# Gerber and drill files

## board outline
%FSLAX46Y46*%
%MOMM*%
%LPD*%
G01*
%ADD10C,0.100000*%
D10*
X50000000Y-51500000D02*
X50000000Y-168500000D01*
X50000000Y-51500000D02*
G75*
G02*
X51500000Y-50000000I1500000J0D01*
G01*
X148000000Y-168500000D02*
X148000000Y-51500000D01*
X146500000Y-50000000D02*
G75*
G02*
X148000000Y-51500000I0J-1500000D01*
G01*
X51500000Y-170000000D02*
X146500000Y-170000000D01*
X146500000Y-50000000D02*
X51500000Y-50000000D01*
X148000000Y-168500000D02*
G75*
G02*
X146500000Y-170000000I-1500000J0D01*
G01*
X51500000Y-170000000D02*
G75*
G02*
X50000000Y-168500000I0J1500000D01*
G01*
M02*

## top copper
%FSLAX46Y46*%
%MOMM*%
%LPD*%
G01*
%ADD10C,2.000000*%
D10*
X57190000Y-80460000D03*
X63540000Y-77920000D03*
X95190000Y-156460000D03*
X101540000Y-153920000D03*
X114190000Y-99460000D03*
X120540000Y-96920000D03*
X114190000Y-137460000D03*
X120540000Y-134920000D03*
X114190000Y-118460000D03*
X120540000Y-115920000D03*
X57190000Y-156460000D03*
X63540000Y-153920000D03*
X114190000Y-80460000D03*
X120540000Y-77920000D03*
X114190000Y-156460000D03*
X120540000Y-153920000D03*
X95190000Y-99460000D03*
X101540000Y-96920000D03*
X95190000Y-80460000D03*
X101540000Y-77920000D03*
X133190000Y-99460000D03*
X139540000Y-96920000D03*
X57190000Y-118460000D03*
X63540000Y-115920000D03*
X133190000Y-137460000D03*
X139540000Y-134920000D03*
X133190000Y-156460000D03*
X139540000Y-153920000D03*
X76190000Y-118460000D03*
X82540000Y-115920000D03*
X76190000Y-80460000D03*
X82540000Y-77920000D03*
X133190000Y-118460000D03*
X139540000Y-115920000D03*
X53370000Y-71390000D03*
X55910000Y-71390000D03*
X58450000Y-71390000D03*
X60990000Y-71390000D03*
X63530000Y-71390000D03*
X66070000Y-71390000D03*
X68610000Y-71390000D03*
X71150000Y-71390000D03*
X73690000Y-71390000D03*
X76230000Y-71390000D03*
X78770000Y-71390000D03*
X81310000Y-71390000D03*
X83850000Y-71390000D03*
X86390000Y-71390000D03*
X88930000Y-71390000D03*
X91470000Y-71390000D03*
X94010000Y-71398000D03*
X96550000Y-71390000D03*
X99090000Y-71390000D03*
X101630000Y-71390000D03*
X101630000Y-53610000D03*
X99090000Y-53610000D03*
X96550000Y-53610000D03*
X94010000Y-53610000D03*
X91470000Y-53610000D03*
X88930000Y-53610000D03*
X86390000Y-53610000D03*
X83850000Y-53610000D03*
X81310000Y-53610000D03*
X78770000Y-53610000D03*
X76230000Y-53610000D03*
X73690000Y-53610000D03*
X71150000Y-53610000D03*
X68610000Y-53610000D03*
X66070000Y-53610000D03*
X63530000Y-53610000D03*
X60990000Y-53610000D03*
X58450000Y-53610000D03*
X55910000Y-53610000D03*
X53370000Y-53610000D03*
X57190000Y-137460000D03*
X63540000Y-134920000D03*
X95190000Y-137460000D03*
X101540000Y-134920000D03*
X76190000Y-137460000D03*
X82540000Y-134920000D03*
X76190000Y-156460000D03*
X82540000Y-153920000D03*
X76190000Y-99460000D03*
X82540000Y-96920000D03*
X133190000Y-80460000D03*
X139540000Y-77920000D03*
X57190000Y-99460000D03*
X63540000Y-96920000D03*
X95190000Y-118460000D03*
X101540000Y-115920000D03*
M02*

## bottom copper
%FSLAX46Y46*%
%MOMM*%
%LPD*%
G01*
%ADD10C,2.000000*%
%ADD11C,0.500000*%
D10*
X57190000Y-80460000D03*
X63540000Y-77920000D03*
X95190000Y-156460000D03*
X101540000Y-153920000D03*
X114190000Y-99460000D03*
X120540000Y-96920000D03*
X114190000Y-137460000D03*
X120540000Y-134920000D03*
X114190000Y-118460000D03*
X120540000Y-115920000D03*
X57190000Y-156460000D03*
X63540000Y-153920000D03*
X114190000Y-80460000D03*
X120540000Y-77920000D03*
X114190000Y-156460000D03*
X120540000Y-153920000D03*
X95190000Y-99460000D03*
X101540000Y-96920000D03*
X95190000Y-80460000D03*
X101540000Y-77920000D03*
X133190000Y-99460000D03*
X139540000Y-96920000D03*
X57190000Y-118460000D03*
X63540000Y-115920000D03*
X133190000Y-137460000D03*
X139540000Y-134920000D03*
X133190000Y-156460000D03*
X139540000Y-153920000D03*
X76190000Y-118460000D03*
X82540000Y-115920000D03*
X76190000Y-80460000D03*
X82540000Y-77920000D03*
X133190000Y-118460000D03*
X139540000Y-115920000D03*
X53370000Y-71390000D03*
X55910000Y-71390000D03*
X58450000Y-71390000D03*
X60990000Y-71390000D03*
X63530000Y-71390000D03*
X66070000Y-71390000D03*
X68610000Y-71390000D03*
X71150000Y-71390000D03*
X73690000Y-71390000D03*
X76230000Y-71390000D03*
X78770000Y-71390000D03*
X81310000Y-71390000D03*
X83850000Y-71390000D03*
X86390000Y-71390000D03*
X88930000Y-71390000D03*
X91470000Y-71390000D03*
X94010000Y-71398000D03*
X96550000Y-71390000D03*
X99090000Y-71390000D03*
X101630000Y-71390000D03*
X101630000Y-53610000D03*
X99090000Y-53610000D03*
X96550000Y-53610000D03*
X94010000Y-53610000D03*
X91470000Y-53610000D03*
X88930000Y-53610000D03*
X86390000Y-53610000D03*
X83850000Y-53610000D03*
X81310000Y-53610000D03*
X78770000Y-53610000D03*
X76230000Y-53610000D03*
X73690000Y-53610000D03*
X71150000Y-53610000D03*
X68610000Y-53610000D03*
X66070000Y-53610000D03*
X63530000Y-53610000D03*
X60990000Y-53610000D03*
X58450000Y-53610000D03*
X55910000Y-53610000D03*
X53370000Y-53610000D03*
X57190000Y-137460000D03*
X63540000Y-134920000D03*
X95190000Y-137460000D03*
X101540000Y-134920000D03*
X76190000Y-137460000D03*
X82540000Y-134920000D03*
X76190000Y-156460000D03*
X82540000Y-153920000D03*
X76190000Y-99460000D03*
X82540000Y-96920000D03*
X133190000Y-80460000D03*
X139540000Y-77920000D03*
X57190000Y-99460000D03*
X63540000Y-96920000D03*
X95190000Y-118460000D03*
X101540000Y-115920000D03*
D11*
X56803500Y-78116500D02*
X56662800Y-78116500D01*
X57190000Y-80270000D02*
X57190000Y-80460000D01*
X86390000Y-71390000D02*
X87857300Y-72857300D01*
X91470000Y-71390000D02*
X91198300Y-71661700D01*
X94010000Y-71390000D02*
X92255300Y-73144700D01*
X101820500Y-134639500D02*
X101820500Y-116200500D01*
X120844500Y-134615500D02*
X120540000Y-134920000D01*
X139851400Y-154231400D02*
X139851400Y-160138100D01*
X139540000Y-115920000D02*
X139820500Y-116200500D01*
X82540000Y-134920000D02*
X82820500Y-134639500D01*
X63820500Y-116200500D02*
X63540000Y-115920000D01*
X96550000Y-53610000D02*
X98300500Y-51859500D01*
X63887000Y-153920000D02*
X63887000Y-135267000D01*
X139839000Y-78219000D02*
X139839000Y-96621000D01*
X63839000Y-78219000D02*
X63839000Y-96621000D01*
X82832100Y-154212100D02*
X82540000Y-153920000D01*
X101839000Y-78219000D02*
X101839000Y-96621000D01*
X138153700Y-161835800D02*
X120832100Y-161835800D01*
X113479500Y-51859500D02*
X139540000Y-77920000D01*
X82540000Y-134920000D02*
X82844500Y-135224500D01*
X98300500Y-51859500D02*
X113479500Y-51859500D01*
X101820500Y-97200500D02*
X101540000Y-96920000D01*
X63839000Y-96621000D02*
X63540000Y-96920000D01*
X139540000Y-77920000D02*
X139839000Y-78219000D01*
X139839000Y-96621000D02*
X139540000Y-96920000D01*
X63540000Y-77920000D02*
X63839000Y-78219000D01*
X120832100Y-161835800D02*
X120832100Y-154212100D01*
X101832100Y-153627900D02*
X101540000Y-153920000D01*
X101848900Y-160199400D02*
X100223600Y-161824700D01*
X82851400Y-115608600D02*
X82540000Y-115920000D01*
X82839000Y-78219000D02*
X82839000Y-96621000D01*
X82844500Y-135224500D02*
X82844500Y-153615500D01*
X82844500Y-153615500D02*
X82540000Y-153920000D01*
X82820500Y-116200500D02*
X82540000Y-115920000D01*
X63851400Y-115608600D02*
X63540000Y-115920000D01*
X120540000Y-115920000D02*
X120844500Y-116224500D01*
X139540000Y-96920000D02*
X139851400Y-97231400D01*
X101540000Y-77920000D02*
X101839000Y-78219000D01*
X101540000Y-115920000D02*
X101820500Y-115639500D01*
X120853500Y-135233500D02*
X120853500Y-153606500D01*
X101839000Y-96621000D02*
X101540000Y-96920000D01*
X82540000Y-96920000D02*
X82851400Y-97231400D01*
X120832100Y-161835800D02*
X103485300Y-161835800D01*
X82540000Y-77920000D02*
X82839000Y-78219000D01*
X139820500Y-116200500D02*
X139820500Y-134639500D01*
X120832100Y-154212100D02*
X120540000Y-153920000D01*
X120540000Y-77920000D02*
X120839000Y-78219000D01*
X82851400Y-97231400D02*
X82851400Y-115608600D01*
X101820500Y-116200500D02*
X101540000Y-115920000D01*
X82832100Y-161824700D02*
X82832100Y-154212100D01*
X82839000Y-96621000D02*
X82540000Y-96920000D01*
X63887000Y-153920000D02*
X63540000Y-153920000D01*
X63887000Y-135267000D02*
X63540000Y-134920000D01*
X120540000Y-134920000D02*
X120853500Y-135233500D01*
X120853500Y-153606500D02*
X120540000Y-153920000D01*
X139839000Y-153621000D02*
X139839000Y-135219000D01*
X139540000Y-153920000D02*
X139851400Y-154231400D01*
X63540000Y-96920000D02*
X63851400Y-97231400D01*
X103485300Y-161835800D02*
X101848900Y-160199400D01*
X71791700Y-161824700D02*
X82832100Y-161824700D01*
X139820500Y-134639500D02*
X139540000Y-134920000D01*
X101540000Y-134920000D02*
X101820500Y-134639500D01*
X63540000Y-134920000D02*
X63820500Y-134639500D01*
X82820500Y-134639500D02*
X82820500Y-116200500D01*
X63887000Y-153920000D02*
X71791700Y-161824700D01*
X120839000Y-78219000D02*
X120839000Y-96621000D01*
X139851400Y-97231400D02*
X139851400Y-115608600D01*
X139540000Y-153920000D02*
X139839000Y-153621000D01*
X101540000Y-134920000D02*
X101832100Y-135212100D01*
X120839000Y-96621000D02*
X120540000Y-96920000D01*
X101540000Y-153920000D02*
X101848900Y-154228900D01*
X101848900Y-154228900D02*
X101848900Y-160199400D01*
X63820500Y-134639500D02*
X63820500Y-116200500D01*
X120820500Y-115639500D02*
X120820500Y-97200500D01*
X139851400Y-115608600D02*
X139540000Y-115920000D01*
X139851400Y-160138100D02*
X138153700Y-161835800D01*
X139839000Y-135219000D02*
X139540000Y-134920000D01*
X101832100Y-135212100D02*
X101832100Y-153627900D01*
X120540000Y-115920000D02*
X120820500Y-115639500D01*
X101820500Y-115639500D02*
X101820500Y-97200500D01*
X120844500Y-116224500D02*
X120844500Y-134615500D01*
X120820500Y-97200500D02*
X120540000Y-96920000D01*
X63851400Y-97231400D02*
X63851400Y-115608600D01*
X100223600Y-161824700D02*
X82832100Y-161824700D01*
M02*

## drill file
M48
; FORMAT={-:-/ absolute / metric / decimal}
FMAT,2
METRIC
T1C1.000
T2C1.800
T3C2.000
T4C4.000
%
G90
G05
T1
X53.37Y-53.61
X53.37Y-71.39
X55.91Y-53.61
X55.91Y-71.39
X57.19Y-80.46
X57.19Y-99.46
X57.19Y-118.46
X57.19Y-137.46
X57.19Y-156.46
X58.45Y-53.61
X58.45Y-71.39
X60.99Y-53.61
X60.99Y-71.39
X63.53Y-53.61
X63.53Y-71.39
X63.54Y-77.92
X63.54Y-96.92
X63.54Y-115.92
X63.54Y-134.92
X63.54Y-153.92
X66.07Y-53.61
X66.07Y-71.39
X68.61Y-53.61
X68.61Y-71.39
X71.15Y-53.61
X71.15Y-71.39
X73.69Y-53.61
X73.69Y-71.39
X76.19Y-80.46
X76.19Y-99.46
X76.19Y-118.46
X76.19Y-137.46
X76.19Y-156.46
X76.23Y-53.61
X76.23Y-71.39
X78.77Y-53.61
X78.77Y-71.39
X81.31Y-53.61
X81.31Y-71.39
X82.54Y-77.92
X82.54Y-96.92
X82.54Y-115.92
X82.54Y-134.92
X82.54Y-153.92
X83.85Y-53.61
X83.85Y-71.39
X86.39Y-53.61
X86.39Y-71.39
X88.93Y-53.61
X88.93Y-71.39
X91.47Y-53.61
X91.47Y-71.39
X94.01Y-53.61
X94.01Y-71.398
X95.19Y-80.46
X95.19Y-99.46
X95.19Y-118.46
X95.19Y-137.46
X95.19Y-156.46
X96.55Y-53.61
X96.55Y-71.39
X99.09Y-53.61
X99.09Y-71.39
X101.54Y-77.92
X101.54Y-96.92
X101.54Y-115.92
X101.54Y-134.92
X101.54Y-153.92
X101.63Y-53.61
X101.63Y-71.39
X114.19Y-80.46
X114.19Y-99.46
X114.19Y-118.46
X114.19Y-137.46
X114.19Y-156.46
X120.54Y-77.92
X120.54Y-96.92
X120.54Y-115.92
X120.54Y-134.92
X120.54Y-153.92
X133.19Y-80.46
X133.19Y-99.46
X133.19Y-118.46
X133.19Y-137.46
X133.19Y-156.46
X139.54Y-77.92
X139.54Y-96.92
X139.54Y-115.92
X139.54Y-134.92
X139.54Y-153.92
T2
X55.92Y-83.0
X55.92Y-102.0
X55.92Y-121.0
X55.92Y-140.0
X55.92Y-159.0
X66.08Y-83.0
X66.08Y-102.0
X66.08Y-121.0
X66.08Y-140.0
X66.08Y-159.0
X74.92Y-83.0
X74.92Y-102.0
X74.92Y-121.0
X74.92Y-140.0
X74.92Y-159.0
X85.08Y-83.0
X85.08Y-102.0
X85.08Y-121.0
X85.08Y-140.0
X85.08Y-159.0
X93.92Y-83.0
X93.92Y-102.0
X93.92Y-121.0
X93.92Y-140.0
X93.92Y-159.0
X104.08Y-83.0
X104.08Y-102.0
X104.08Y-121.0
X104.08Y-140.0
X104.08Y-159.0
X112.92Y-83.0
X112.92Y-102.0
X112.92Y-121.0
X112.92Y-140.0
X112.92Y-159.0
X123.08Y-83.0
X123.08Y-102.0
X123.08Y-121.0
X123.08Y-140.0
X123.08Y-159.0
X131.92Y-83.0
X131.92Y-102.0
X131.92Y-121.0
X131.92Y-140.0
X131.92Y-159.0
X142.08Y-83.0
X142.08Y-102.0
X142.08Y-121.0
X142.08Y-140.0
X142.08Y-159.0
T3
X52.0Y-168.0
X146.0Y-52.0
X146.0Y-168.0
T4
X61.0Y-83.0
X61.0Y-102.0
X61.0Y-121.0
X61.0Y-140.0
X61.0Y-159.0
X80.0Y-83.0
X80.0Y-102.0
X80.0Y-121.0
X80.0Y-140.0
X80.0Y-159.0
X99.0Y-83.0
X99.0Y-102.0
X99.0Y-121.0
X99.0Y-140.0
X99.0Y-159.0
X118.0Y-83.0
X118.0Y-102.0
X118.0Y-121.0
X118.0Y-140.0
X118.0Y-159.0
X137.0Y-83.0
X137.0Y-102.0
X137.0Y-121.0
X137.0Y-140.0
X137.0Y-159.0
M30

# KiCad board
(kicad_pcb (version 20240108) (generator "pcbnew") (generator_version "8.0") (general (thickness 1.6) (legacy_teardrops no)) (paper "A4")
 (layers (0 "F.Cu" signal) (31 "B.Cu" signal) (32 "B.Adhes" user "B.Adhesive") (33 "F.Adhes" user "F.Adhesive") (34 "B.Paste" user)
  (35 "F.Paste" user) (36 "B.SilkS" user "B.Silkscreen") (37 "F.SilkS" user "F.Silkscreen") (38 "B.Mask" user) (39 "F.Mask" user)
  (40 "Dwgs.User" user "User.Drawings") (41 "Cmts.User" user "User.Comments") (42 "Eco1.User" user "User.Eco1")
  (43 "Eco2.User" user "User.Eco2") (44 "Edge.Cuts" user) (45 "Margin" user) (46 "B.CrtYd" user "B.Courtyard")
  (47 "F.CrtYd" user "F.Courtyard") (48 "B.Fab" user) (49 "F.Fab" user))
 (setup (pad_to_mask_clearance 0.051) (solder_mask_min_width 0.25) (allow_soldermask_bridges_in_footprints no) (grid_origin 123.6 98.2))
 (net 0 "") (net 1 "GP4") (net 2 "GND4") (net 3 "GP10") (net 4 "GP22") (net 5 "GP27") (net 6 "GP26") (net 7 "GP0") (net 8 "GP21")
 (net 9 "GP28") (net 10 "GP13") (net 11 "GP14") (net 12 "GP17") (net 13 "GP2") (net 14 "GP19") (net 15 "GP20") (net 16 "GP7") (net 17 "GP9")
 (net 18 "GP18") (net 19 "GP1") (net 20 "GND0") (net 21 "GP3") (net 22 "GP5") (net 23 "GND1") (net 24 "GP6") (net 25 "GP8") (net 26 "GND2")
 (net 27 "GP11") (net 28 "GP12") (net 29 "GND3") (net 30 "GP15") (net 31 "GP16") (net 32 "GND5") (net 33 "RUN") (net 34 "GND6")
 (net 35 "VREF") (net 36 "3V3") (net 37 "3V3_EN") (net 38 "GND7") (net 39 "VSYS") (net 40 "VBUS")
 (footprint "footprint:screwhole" (layer "F.Cu") (at 146 52)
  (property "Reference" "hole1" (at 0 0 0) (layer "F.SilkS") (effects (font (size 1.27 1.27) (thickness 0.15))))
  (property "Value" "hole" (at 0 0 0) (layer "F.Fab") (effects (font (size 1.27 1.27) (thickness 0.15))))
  (pad "" np_thru_hole circle (at 0 0) (size 2 2) (drill 2) (layers "*.Cu" "*.Mask")))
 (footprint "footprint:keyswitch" (layer "F.Cu") (at 61 83)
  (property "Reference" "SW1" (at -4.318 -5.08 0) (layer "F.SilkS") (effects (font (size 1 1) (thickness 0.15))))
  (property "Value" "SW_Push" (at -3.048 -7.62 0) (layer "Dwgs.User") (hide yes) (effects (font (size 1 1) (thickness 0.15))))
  (pad "" np_thru_hole circle (at -5.08 0) (size 1.8 1.8) (drill 1.8) (layers "*.Cu" "*.Mask"))
  (pad "" np_thru_hole circle (at 0 0) (size 4 4) (drill 4) (layers "*.Cu" "*.Mask"))
  (pad "" np_thru_hole circle (at 5.08 0) (size 1.8 1.8) (drill 1.8) (layers "*.Cu" "*.Mask"))
  (pad "1" thru_hole circle (at -3.81 -2.54) (size 2 2) (drill 1) (layers "*.Cu" "*.Mask") (remove_unused_layers no) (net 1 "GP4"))
  (pad "2" thru_hole circle (at 2.54 -5.08) (size 2 2) (drill 1) (layers "*.Cu" "*.Mask") (remove_unused_layers no) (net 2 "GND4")))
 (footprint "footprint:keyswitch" (layer "F.Cu") (at 99 159)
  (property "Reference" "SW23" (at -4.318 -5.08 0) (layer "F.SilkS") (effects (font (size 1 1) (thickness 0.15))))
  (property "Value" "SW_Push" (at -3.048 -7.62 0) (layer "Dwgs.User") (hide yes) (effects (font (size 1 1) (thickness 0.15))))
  (pad "" np_thru_hole circle (at -5.08 0) (size 1.8 1.8) (drill 1.8) (layers "*.Cu" "*.Mask"))
  (pad "" np_thru_hole circle (at 0 0) (size 4 4) (drill 4) (layers "*.Cu" "*.Mask"))
  (pad "" np_thru_hole circle (at 5.08 0) (size 1.8 1.8) (drill 1.8) (layers "*.Cu" "*.Mask"))
  (pad "1" thru_hole circle (at -3.81 -2.54) (size 2 2) (drill 1) (layers "*.Cu" "*.Mask") (remove_unused_layers no) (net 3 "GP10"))
  (pad "2" thru_hole circle (at 2.54 -5.08) (size 2 2) (drill 1) (layers "*.Cu" "*.Mask") (remove_unused_layers no) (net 2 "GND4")))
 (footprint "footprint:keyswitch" (layer "F.Cu") (at 118 102)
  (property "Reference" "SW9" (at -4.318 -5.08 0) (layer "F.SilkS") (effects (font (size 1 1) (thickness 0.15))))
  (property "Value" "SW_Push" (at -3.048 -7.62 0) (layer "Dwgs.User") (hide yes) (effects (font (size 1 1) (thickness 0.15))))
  (pad "" np_thru_hole circle (at -5.08 0) (size 1.8 1.8) (drill 1.8) (layers "*.Cu" "*.Mask"))
  (pad "" np_thru_hole circle (at 0 0) (size 4 4) (drill 4) (layers "*.Cu" "*.Mask"))
  (pad "" np_thru_hole circle (at 5.08 0) (size 1.8 1.8) (drill 1.8) (layers "*.Cu" "*.Mask"))
  (pad "1" thru_hole circle (at -3.81 -2.54) (size 2 2) (drill 1) (layers "*.Cu" "*.Mask") (remove_unused_layers no) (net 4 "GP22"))
  (pad "2" thru_hole circle (at 2.54 -5.08) (size 2 2) (drill 1) (layers "*.Cu" "*.Mask") (remove_unused_layers no) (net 2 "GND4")))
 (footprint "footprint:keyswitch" (layer "F.Cu") (at 118 140)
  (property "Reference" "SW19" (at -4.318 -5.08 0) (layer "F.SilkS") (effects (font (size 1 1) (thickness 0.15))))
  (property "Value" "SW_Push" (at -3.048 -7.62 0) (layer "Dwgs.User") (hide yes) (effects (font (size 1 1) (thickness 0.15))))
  (pad "" np_thru_hole circle (at -5.08 0) (size 1.8 1.8) (drill 1.8) (layers "*.Cu" "*.Mask"))
  (pad "" np_thru_hole circle (at 0 0) (size 4 4) (drill 4) (layers "*.Cu" "*.Mask"))
  (pad "" np_thru_hole circle (at 5.08 0) (size 1.8 1.8) (drill 1.8) (layers "*.Cu" "*.Mask"))
  (pad "1" thru_hole circle (at -3.81 -2.54) (size 2 2) (drill 1) (layers "*.Cu" "*.Mask") (remove_unused_layers no) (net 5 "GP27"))
  (pad "2" thru_hole circle (at 2.54 -5.08) (size 2 2) (drill 1) (layers "*.Cu" "*.Mask") (remove_unused_layers no) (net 2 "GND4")))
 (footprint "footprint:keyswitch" (layer "F.Cu") (at 118 121)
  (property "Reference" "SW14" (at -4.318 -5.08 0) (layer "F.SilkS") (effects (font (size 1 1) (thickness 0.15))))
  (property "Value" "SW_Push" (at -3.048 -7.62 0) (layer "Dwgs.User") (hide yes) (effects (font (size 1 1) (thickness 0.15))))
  (pad "" np_thru_hole circle (at -5.08 0) (size 1.8 1.8) (drill 1.8) (layers "*.Cu" "*.Mask"))
  (pad "" np_thru_hole circle (at 0 0) (size 4 4) (drill 4) (layers "*.Cu" "*.Mask"))
  (pad "" np_thru_hole circle (at 5.08 0) (size 1.8 1.8) (drill 1.8) (layers "*.Cu" "*.Mask"))
  (pad "1" thru_hole circle (at -3.81 -2.54) (size 2 2) (drill 1) (layers "*.Cu" "*.Mask") (remove_unused_layers no) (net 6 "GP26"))
  (pad "2" thru_hole circle (at 2.54 -5.08) (size 2 2) (drill 1) (layers "*.Cu" "*.Mask") (remove_unused_layers no) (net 2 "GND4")))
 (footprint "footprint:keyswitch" (layer "F.Cu") (at 61 159)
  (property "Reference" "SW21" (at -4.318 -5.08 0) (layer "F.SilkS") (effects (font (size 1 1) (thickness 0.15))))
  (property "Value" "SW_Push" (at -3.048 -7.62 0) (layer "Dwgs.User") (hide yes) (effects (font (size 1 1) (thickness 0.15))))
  (pad "" np_thru_hole circle (at -5.08 0) (size 1.8 1.8) (drill 1.8) (layers "*.Cu" "*.Mask"))
  (pad "" np_thru_hole circle (at 0 0) (size 4 4) (drill 4) (layers "*.Cu" "*.Mask"))
  (pad "" np_thru_hole circle (at 5.08 0) (size 1.8 1.8) (drill 1.8) (layers "*.Cu" "*.Mask"))
  (pad "1" thru_hole circle (at -3.81 -2.54) (size 2 2) (drill 1) (layers "*.Cu" "*.Mask") (remove_unused_layers no) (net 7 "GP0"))
  (pad "2" thru_hole circle (at 2.54 -5.08) (size 2 2) (drill 1) (layers "*.Cu" "*.Mask") (remove_unused_layers no) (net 2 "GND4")))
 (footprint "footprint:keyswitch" (layer "F.Cu") (at 118 83)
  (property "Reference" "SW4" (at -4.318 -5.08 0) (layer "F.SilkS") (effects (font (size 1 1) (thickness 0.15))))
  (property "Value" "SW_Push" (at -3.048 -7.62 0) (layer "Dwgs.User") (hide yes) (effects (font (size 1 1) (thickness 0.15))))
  (pad "" np_thru_hole circle (at -5.08 0) (size 1.8 1.8) (drill 1.8) (layers "*.Cu" "*.Mask"))
  (pad "" np_thru_hole circle (at 0 0) (size 4 4) (drill 4) (layers "*.Cu" "*.Mask"))
  (pad "" np_thru_hole circle (at 5.08 0) (size 1.8 1.8) (drill 1.8) (layers "*.Cu" "*.Mask"))
  (pad "1" thru_hole circle (at -3.81 -2.54) (size 2 2) (drill 1) (layers "*.Cu" "*.Mask") (remove_unused_layers no) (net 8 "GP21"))
  (pad "2" thru_hole circle (at 2.54 -5.08) (size 2 2) (drill 1) (layers "*.Cu" "*.Mask") (remove_unused_layers no) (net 2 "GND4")))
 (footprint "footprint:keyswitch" (layer "F.Cu") (at 118 159)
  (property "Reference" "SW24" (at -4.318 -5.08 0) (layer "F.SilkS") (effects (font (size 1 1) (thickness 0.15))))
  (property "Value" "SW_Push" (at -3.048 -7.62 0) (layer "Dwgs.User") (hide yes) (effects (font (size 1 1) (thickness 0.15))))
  (pad "" np_thru_hole circle (at -5.08 0) (size 1.8 1.8) (drill 1.8) (layers "*.Cu" "*.Mask"))
  (pad "" np_thru_hole circle (at 0 0) (size 4 4) (drill 4) (layers "*.Cu" "*.Mask"))
  (pad "" np_thru_hole circle (at 5.08 0) (size 1.8 1.8) (drill 1.8) (layers "*.Cu" "*.Mask"))
  (pad "1" thru_hole circle (at -3.81 -2.54) (size 2 2) (drill 1) (layers "*.Cu" "*.Mask") (remove_unused_layers no) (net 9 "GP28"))
  (pad "2" thru_hole circle (at 2.54 -5.08) (size 2 2) (drill 1) (layers "*.Cu" "*.Mask") (remove_unused_layers no) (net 2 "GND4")))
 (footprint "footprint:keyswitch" (layer "F.Cu") (at 99 102)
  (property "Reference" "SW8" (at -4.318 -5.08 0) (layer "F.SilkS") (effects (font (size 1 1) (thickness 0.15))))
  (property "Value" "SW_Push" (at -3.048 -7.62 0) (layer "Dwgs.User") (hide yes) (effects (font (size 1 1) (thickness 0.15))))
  (pad "" np_thru_hole circle (at -5.08 0) (size 1.8 1.8) (drill 1.8) (layers "*.Cu" "*.Mask"))
  (pad "" np_thru_hole circle (at 0 0) (size 4 4) (drill 4) (layers "*.Cu" "*.Mask"))
  (pad "" np_thru_hole circle (at 5.08 0) (size 1.8 1.8) (drill 1.8) (layers "*.Cu" "*.Mask"))
  (pad "1" thru_hole circle (at -3.81 -2.54) (size 2 2) (drill 1) (layers "*.Cu" "*.Mask") (remove_unused_layers no) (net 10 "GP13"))
  (pad "2" thru_hole circle (at 2.54 -5.08) (size 2 2) (drill 1) (layers "*.Cu" "*.Mask") (remove_unused_layers no) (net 2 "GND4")))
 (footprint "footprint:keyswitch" (layer "F.Cu") (at 99 83)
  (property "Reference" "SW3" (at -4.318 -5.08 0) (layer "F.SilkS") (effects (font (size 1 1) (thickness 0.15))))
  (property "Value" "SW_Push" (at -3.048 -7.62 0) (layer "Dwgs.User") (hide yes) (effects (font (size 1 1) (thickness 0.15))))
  (pad "" np_thru_hole circle (at -5.08 0) (size 1.8 1.8) (drill 1.8) (layers "*.Cu" "*.Mask"))
  (pad "" np_thru_hole circle (at 0 0) (size 4 4) (drill 4) (layers "*.Cu" "*.Mask"))
  (pad "" np_thru_hole circle (at 5.08 0) (size 1.8 1.8) (drill 1.8) (layers "*.Cu" "*.Mask"))
  (pad "1" thru_hole circle (at -3.81 -2.54) (size 2 2) (drill 1) (layers "*.Cu" "*.Mask") (remove_unused_layers no) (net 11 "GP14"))
  (pad "2" thru_hole circle (at 2.54 -5.08) (size 2 2) (drill 1) (layers "*.Cu" "*.Mask") (remove_unused_layers no) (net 2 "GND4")))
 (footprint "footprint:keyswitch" (layer "F.Cu") (at 137 102)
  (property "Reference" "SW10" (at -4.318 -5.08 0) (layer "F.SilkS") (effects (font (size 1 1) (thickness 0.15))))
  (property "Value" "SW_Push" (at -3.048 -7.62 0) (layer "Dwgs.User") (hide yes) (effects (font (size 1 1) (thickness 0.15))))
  (pad "" np_thru_hole circle (at -5.08 0) (size 1.8 1.8) (drill 1.8) (layers "*.Cu" "*.Mask"))
  (pad "" np_thru_hole circle (at 0 0) (size 4 4) (drill 4) (layers "*.Cu" "*.Mask"))
  (pad "" np_thru_hole circle (at 5.08 0) (size 1.8 1.8) (drill 1.8) (layers "*.Cu" "*.Mask"))
  (pad "1" thru_hole circle (at -3.81 -2.54) (size 2 2) (drill 1) (layers "*.Cu" "*.Mask") (remove_unused_layers no) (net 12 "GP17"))
  (pad "2" thru_hole circle (at 2.54 -5.08) (size 2 2) (drill 1) (layers "*.Cu" "*.Mask") (remove_unused_layers no) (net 2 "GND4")))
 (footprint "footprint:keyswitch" (layer "F.Cu") (at 61 121)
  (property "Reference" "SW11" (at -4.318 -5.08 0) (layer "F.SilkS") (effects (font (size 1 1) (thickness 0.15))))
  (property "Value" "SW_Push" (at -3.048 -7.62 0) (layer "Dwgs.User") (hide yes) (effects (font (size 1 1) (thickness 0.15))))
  (pad "" np_thru_hole circle (at -5.08 0) (size 1.8 1.8) (drill 1.8) (layers "*.Cu" "*.Mask"))
  (pad "" np_thru_hole circle (at 0 0) (size 4 4) (drill 4) (layers "*.Cu" "*.Mask"))
  (pad "" np_thru_hole circle (at 5.08 0) (size 1.8 1.8) (drill 1.8) (layers "*.Cu" "*.Mask"))
  (pad "1" thru_hole circle (at -3.81 -2.54) (size 2 2) (drill 1) (layers "*.Cu" "*.Mask") (remove_unused_layers no) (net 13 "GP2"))
  (pad "2" thru_hole circle (at 2.54 -5.08) (size 2 2) (drill 1) (layers "*.Cu" "*.Mask") (remove_unused_layers no) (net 2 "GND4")))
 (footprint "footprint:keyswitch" (layer "F.Cu") (at 137 140)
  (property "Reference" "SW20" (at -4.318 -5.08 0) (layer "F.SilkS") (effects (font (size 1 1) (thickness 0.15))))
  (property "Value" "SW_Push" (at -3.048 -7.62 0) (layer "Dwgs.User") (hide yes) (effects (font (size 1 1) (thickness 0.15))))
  (pad "" np_thru_hole circle (at -5.08 0) (size 1.8 1.8) (drill 1.8) (layers "*.Cu" "*.Mask"))
  (pad "" np_thru_hole circle (at 0 0) (size 4 4) (drill 4) (layers "*.Cu" "*.Mask"))
  (pad "" np_thru_hole circle (at 5.08 0) (size 1.8 1.8) (drill 1.8) (layers "*.Cu" "*.Mask"))
  (pad "1" thru_hole circle (at -3.81 -2.54) (size 2 2) (drill 1) (layers "*.Cu" "*.Mask") (remove_unused_layers no) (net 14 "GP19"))
  (pad "2" thru_hole circle (at 2.54 -5.08) (size 2 2) (drill 1) (layers "*.Cu" "*.Mask") (remove_unused_layers no) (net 2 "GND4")))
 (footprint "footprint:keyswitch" (layer "F.Cu") (at 137 159)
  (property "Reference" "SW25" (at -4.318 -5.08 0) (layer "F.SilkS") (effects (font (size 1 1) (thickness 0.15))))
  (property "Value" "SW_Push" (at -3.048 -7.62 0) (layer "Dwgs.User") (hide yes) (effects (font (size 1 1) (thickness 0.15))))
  (pad "" np_thru_hole circle (at -5.08 0) (size 1.8 1.8) (drill 1.8) (layers "*.Cu" "*.Mask"))
  (pad "" np_thru_hole circle (at 0 0) (size 4 4) (drill 4) (layers "*.Cu" "*.Mask"))
  (pad "" np_thru_hole circle (at 5.08 0) (size 1.8 1.8) (drill 1.8) (layers "*.Cu" "*.Mask"))
  (pad "1" thru_hole circle (at -3.81 -2.54) (size 2 2) (drill 1) (layers "*.Cu" "*.Mask") (remove_unused_layers no) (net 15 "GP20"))
  (pad "2" thru_hole circle (at 2.54 -5.08) (size 2 2) (drill 1) (layers "*.Cu" "*.Mask") (remove_unused_layers no) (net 2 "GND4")))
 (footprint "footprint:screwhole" (layer "F.Cu") (at 52 168)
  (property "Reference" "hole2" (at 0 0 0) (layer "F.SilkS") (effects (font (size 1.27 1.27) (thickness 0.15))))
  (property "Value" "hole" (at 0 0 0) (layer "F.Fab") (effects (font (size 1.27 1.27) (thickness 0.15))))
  (pad "" np_thru_hole circle (at 0 0) (size 2 2) (drill 2) (layers "*.Cu" "*.Mask")))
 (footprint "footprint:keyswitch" (layer "F.Cu") (at 80 121)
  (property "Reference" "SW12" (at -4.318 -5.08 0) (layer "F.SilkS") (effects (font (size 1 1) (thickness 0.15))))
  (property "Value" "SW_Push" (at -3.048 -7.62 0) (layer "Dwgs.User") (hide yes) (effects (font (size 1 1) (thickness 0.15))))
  (pad "" np_thru_hole circle (at -5.08 0) (size 1.8 1.8) (drill 1.8) (layers "*.Cu" "*.Mask"))
  (pad "" np_thru_hole circle (at 0 0) (size 4 4) (drill 4) (layers "*.Cu" "*.Mask"))
  (pad "" np_thru_hole circle (at 5.08 0) (size 1.8 1.8) (drill 1.8) (layers "*.Cu" "*.Mask"))
  (pad "1" thru_hole circle (at -3.81 -2.54) (size 2 2) (drill 1) (layers "*.Cu" "*.Mask") (remove_unused_layers no) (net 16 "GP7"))
  (pad "2" thru_hole circle (at 2.54 -5.08) (size 2 2) (drill 1) (layers "*.Cu" "*.Mask") (remove_unused_layers no) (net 2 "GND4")))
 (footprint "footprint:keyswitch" (layer "F.Cu") (at 80 83)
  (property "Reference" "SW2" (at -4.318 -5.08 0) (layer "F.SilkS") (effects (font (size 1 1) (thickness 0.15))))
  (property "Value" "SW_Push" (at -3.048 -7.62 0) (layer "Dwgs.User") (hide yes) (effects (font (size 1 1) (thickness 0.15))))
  (pad "" np_thru_hole circle (at -5.08 0) (size 1.8 1.8) (drill 1.8) (layers "*.Cu" "*.Mask"))
  (pad "" np_thru_hole circle (at 0 0) (size 4 4) (drill 4) (layers "*.Cu" "*.Mask"))
  (pad "" np_thru_hole circle (at 5.08 0) (size 1.8 1.8) (drill 1.8) (layers "*.Cu" "*.Mask"))
  (pad "1" thru_hole circle (at -3.81 -2.54) (size 2 2) (drill 1) (layers "*.Cu" "*.Mask") (remove_unused_layers no) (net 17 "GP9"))
  (pad "2" thru_hole circle (at 2.54 -5.08) (size 2 2) (drill 1) (layers "*.Cu" "*.Mask") (remove_unused_layers no) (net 2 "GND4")))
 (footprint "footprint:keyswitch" (layer "F.Cu") (at 137 121)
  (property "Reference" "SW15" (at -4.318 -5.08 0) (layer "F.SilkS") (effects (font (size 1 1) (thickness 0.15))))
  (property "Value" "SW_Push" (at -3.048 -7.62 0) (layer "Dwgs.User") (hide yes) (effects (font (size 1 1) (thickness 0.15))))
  (pad "" np_thru_hole circle (at -5.08 0) (size 1.8 1.8) (drill 1.8) (layers "*.Cu" "*.Mask"))
  (pad "" np_thru_hole circle (at 0 0) (size 4 4) (drill 4) (layers "*.Cu" "*.Mask"))
  (pad "" np_thru_hole circle (at 5.08 0) (size 1.8 1.8) (drill 1.8) (layers "*.Cu" "*.Mask"))
  (pad "1" thru_hole circle (at -3.81 -2.54) (size 2 2) (drill 1) (layers "*.Cu" "*.Mask") (remove_unused_layers no) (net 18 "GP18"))
  (pad "2" thru_hole circle (at 2.54 -5.08) (size 2 2) (drill 1) (layers "*.Cu" "*.Mask") (remove_unused_layers no) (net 2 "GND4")))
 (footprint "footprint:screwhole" (layer "F.Cu") (at 146 168)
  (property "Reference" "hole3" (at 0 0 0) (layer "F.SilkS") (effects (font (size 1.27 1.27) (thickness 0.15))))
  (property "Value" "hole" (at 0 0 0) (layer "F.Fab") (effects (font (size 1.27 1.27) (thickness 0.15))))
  (pad "" np_thru_hole circle (at 0 0) (size 2 2) (drill 2) (layers "*.Cu" "*.Mask")))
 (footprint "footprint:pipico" (layer "F.Cu") (at 77.5 62.5)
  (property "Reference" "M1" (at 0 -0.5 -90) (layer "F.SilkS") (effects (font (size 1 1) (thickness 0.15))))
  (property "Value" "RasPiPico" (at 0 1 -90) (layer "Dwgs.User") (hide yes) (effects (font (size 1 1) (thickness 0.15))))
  (pad "1" thru_hole circle (at -24.13 8.89 270) (size 2 2) (drill 1) (layers "*.Cu" "*.Mask") (remove_unused_layers no) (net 7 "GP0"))
  (pad "2" thru_hole circle (at -21.59 8.89 270) (size 2 2) (drill 1) (layers "*.Cu" "*.Mask") (remove_unused_layers no) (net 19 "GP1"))
  (pad "3" thru_hole circle (at -19.05 8.89 270) (size 2 2) (drill 1) (layers "*.Cu" "*.Mask") (remove_unused_layers no) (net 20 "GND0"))
  (pad "4" thru_hole circle (at -16.51 8.89 270) (size 2 2) (drill 1) (layers "*.Cu" "*.Mask") (remove_unused_layers no) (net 13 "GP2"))
  (pad "5" thru_hole circle (at -13.97 8.89 270) (size 2 2) (drill 1) (layers "*.Cu" "*.Mask") (remove_unused_layers no) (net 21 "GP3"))
  (pad "6" thru_hole circle (at -11.43 8.89 270) (size 2 2) (drill 1) (layers "*.Cu" "*.Mask") (remove_unused_layers no) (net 1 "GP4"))
  (pad "7" thru_hole circle (at -8.89 8.89 270) (size 2 2) (drill 1) (layers "*.Cu" "*.Mask") (remove_unused_layers no) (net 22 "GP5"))
  (pad "8" thru_hole circle (at -6.35 8.89 270) (size 2 2) (drill 1) (layers "*.Cu" "*.Mask") (remove_unused_layers no) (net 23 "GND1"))
  (pad "9" thru_hole circle (at -3.81 8.89 270) (size 2 2) (drill 1) (layers "*.Cu" "*.Mask") (remove_unused_layers no) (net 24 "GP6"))
  (pad "10" thru_hole circle (at -1.27 8.89 270) (size 2 2) (drill 1) (layers "*.Cu" "*.Mask") (remove_unused_layers no) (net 16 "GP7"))
  (pad "11" thru_hole circle (at 1.27 8.89 270) (size 2 2) (drill 1) (layers "*.Cu" "*.Mask") (remove_unused_layers no) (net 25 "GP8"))
  (pad "12" thru_hole circle (at 3.81 8.89 270) (size 2 2) (drill 1) (layers "*.Cu" "*.Mask") (remove_unused_layers no) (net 17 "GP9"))
  (pad "13" thru_hole circle (at 6.35 8.89 270) (size 2 2) (drill 1) (layers "*.Cu" "*.Mask") (remove_unused_layers no) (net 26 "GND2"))
  (pad "14" thru_hole circle (at 8.89 8.89 270) (size 2 2) (drill 1) (layers "*.Cu" "*.Mask") (remove_unused_layers no) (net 3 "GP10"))
  (pad "15" thru_hole circle (at 11.43 8.89 270) (size 2 2) (drill 1) (layers "*.Cu" "*.Mask") (remove_unused_layers no) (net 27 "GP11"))
  (pad "16" thru_hole circle (at 13.97 8.89 270) (size 2 2) (drill 1) (layers "*.Cu" "*.Mask") (remove_unused_layers no) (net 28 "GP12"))
  (pad "17" thru_hole circle (at 16.51 8.898 270) (size 2 2) (drill 1) (layers "*.Cu" "*.Mask") (remove_unused_layers no) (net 10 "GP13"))
  (pad "18" thru_hole circle (at 19.05 8.89 270) (size 2 2) (drill 1) (layers "*.Cu" "*.Mask") (remove_unused_layers no) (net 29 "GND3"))
  (pad "19" thru_hole circle (at 21.59 8.89 270) (size 2 2) (drill 1) (layers "*.Cu" "*.Mask") (remove_unused_layers no) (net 11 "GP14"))
  (pad "20" thru_hole circle (at 24.13 8.89 270) (size 2 2) (drill 1) (layers "*.Cu" "*.Mask") (remove_unused_layers no) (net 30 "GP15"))
  (pad "21" thru_hole circle (at 24.13 -8.89 270) (size 2 2) (drill 1) (layers "*.Cu" "*.Mask") (remove_unused_layers no) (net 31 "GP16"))
  (pad "22" thru_hole circle (at 21.59 -8.89 270) (size 2 2) (drill 1) (layers "*.Cu" "*.Mask") (remove_unused_layers no) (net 12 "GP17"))
  (pad "23" thru_hole circle (at 19.05 -8.89 270) (size 2 2) (drill 1) (layers "*.Cu" "*.Mask") (remove_unused_layers no) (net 2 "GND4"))
  (pad "24" thru_hole circle (at 16.51 -8.89 270) (size 2 2) (drill 1) (layers "*.Cu" "*.Mask") (remove_unused_layers no) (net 18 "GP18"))
  (pad "25" thru_hole circle (at 13.97 -8.89 270) (size 2 2) (drill 1) (layers "*.Cu" "*.Mask") (remove_unused_layers no) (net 14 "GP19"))
  (pad "26" thru_hole circle (at 11.43 -8.89 270) (size 2 2) (drill 1) (layers "*.Cu" "*.Mask") (remove_unused_layers no) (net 15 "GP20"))
  (pad "27" thru_hole circle (at 8.89 -8.89 270) (size 2 2) (drill 1) (layers "*.Cu" "*.Mask") (remove_unused_layers no) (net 8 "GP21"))
  (pad "28" thru_hole circle (at 6.35 -8.89 270) (size 2 2) (drill 1) (layers "*.Cu" "*.Mask") (remove_unused_layers no) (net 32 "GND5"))
  (pad "29" thru_hole circle (at 3.81 -8.89 270) (size 2 2) (drill 1) (layers "*.Cu" "*.Mask") (remove_unused_layers no) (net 4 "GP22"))
  (pad "30" thru_hole circle (at 1.27 -8.89 270) (size 2 2) (drill 1) (layers "*.Cu" "*.Mask") (remove_unused_layers no) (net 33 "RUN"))
  (pad "31" thru_hole circle (at -1.27 -8.89 270) (size 2 2) (drill 1) (layers "*.Cu" "*.Mask") (remove_unused_layers no) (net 6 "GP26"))
  (pad "32" thru_hole circle (at -3.81 -8.89 270) (size 2 2) (drill 1) (layers "*.Cu" "*.Mask") (remove_unused_layers no) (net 5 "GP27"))
  (pad "33" thru_hole circle (at -6.35 -8.89 270) (size 2 2) (drill 1) (layers "*.Cu" "*.Mask") (remove_unused_layers no) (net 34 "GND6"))
  (pad "34" thru_hole circle (at -8.89 -8.89 270) (size 2 2) (drill 1) (layers "*.Cu" "*.Mask") (remove_unused_layers no) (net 9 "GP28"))
  (pad "35" thru_hole circle (at -11.43 -8.89 270) (size 2 2) (drill 1) (layers "*.Cu" "*.Mask") (remove_unused_layers no) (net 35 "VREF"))
  (pad "36" thru_hole circle (at -13.97 -8.89 270) (size 2 2) (drill 1) (layers "*.Cu" "*.Mask") (remove_unused_layers no) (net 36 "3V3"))
  (pad "37" thru_hole circle (at -16.51 -8.89 270) (size 2 2) (drill 1) (layers "*.Cu" "*.Mask") (remove_unused_layers no) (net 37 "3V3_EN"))
  (pad "38" thru_hole circle (at -19.05 -8.89 270) (size 2 2) (drill 1) (layers "*.Cu" "*.Mask") (remove_unused_layers no) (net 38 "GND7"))
  (pad "39" thru_hole circle (at -21.59 -8.89 270) (size 2 2) (drill 1) (layers "*.Cu" "*.Mask") (remove_unused_layers no) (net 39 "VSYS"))
  (pad "40" thru_hole circle (at -24.13 -8.89 270) (size 2 2) (drill 1) (layers "*.Cu" "*.Mask") (remove_unused_layers no) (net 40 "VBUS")))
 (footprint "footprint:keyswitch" (layer "F.Cu") (at 61 140)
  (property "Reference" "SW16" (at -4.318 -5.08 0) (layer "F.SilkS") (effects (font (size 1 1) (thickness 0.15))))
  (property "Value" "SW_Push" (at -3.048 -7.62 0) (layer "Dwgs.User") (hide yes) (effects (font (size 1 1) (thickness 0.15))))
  (pad "" np_thru_hole circle (at -5.08 0) (size 1.8 1.8) (drill 1.8) (layers "*.Cu" "*.Mask"))
  (pad "" np_thru_hole circle (at 0 0) (size 4 4) (drill 4) (layers "*.Cu" "*.Mask"))
  (pad "" np_thru_hole circle (at 5.08 0) (size 1.8 1.8) (drill 1.8) (layers "*.Cu" "*.Mask"))
  (pad "1" thru_hole circle (at -3.81 -2.54) (size 2 2) (drill 1) (layers "*.Cu" "*.Mask") (remove_unused_layers no) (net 19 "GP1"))
  (pad "2" thru_hole circle (at 2.54 -5.08) (size 2 2) (drill 1) (layers "*.Cu" "*.Mask") (remove_unused_layers no) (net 2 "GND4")))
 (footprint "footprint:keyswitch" (layer "F.Cu") (at 99 140)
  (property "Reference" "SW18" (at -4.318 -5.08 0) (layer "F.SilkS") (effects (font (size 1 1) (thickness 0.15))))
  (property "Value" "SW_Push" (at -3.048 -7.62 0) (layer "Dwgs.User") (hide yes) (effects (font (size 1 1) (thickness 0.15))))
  (pad "" np_thru_hole circle (at -5.08 0) (size 1.8 1.8) (drill 1.8) (layers "*.Cu" "*.Mask"))
  (pad "" np_thru_hole circle (at 0 0) (size 4 4) (drill 4) (layers "*.Cu" "*.Mask"))
  (pad "" np_thru_hole circle (at 5.08 0) (size 1.8 1.8) (drill 1.8) (layers "*.Cu" "*.Mask"))
  (pad "1" thru_hole circle (at -3.81 -2.54) (size 2 2) (drill 1) (layers "*.Cu" "*.Mask") (remove_unused_layers no) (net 27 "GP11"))
  (pad "2" thru_hole circle (at 2.54 -5.08) (size 2 2) (drill 1) (layers "*.Cu" "*.Mask") (remove_unused_layers no) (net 2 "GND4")))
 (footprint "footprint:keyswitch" (layer "F.Cu") (at 80 140)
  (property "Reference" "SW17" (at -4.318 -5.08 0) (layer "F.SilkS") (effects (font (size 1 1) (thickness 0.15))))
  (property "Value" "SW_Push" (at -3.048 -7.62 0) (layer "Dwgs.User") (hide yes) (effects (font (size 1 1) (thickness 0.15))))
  (pad "" np_thru_hole circle (at -5.08 0) (size 1.8 1.8) (drill 1.8) (layers "*.Cu" "*.Mask"))
  (pad "" np_thru_hole circle (at 0 0) (size 4 4) (drill 4) (layers "*.Cu" "*.Mask"))
  (pad "" np_thru_hole circle (at 5.08 0) (size 1.8 1.8) (drill 1.8) (layers "*.Cu" "*.Mask"))
  (pad "1" thru_hole circle (at -3.81 -2.54) (size 2 2) (drill 1) (layers "*.Cu" "*.Mask") (remove_unused_layers no) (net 24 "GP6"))
  (pad "2" thru_hole circle (at 2.54 -5.08) (size 2 2) (drill 1) (layers "*.Cu" "*.Mask") (remove_unused_layers no) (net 2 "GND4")))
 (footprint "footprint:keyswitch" (layer "F.Cu") (at 80 159)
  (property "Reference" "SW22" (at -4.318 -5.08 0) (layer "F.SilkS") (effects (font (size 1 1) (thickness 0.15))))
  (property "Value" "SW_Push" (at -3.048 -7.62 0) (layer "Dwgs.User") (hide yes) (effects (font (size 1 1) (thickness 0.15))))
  (pad "" np_thru_hole circle (at -5.08 0) (size 1.8 1.8) (drill 1.8) (layers "*.Cu" "*.Mask"))
  (pad "" np_thru_hole circle (at 0 0) (size 4 4) (drill 4) (layers "*.Cu" "*.Mask"))
  (pad "" np_thru_hole circle (at 5.08 0) (size 1.8 1.8) (drill 1.8) (layers "*.Cu" "*.Mask"))
  (pad "1" thru_hole circle (at -3.81 -2.54) (size 2 2) (drill 1) (layers "*.Cu" "*.Mask") (remove_unused_layers no) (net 22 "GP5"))
  (pad "2" thru_hole circle (at 2.54 -5.08) (size 2 2) (drill 1) (layers "*.Cu" "*.Mask") (remove_unused_layers no) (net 2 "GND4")))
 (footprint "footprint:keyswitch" (layer "F.Cu") (at 80 102)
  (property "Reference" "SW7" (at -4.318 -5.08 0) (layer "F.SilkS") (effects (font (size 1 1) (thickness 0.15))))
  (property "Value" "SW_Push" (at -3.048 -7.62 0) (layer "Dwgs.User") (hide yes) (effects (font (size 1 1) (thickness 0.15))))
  (pad "" np_thru_hole circle (at -5.08 0) (size 1.8 1.8) (drill 1.8) (layers "*.Cu" "*.Mask"))
  (pad "" np_thru_hole circle (at 0 0) (size 4 4) (drill 4) (layers "*.Cu" "*.Mask"))
  (pad "" np_thru_hole circle (at 5.08 0) (size 1.8 1.8) (drill 1.8) (layers "*.Cu" "*.Mask"))
  (pad "1" thru_hole circle (at -3.81 -2.54) (size 2 2) (drill 1) (layers "*.Cu" "*.Mask") (remove_unused_layers no) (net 25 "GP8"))
  (pad "2" thru_hole circle (at 2.54 -5.08) (size 2 2) (drill 1) (layers "*.Cu" "*.Mask") (remove_unused_layers no) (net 2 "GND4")))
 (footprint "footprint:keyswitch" (layer "F.Cu") (at 137 83)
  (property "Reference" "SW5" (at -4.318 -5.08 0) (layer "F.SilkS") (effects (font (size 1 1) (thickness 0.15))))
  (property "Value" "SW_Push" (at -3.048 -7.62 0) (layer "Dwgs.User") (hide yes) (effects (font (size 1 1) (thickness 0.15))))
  (pad "" np_thru_hole circle (at -5.08 0) (size 1.8 1.8) (drill 1.8) (layers "*.Cu" "*.Mask"))
  (pad "" np_thru_hole circle (at 0 0) (size 4 4) (drill 4) (layers "*.Cu" "*.Mask"))
  (pad "" np_thru_hole circle (at 5.08 0) (size 1.8 1.8) (drill 1.8) (layers "*.Cu" "*.Mask"))
  (pad "1" thru_hole circle (at -3.81 -2.54) (size 2 2) (drill 1) (layers "*.Cu" "*.Mask") (remove_unused_layers no) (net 31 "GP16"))
  (pad "2" thru_hole circle (at 2.54 -5.08) (size 2 2) (drill 1) (layers "*.Cu" "*.Mask") (remove_unused_layers no) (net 2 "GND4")))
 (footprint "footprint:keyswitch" (layer "F.Cu") (at 61 102)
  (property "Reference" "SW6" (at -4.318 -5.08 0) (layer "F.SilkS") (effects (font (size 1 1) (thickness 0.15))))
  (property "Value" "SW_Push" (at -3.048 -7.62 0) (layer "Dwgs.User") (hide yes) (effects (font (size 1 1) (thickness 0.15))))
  (pad "" np_thru_hole circle (at -5.08 0) (size 1.8 1.8) (drill 1.8) (layers "*.Cu" "*.Mask"))
  (pad "" np_thru_hole circle (at 0 0) (size 4 4) (drill 4) (layers "*.Cu" "*.Mask"))
  (pad "" np_thru_hole circle (at 5.08 0) (size 1.8 1.8) (drill 1.8) (layers "*.Cu" "*.Mask"))
  (pad "1" thru_hole circle (at -3.81 -2.54) (size 2 2) (drill 1) (layers "*.Cu" "*.Mask") (remove_unused_layers no) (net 21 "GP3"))
  (pad "2" thru_hole circle (at 2.54 -5.08) (size 2 2) (drill 1) (layers "*.Cu" "*.Mask") (remove_unused_layers no) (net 2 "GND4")))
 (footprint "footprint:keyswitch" (layer "F.Cu") (at 99 121)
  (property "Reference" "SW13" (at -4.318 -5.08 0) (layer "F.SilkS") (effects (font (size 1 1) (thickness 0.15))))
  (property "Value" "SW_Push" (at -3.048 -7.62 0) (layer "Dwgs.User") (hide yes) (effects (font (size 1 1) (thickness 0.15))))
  (pad "" np_thru_hole circle (at -5.08 0) (size 1.8 1.8) (drill 1.8) (layers "*.Cu" "*.Mask"))
  (pad "" np_thru_hole circle (at 0 0) (size 4 4) (drill 4) (layers "*.Cu" "*.Mask"))
  (pad "" np_thru_hole circle (at 5.08 0) (size 1.8 1.8) (drill 1.8) (layers "*.Cu" "*.Mask"))
  (pad "1" thru_hole circle (at -3.81 -2.54) (size 2 2) (drill 1) (layers "*.Cu" "*.Mask") (remove_unused_layers no) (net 28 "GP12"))
  (pad "2" thru_hole circle (at 2.54 -5.08) (size 2 2) (drill 1) (layers "*.Cu" "*.Mask") (remove_unused_layers no) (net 2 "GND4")))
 (gr_line (start 50 51.5) (end 50 168.5) (stroke (width 0.1) (type solid)) (layer "Edge.Cuts"))
 (gr_arc (start 50 51.5) (mid 50.43934 50.43934) (end 51.5 50) (stroke (width 0.1) (type solid)) (layer "Edge.Cuts"))
 (gr_line (start 148 168.5) (end 148 51.5) (stroke (width 0.1) (type solid)) (layer "Edge.Cuts"))
 (gr_arc (start 146.5 50) (mid 147.56066 50.43934) (end 148 51.5) (stroke (width 0.1) (type solid)) (layer "Edge.Cuts"))
 (gr_line (start 51.5 170) (end 146.5 170) (stroke (width 0.1) (type solid)) (layer "Edge.Cuts"))
 (gr_line (start 146.5 50) (end 51.5 50) (stroke (width 0.1) (type solid)) (layer "Edge.Cuts"))
 (gr_arc (start 148 168.5) (mid 147.56066 169.56066) (end 146.5 170) (stroke (width 0.1) (type solid)) (layer "Edge.Cuts"))
 (gr_arc (start 51.5 170) (mid 50.43934 169.56066) (end 50 168.5) (stroke (width 0.1) (type solid)) (layer "Edge.Cuts"))
 (segment (start 56.8035 78.1165) (end 56.6628 78.1165) (width 0.5) (layer "B.Cu") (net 21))
 (segment (start 57.19 80.27) (end 57.19 80.46) (width 0.5) (layer "B.Cu") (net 1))
 (segment (start 86.39 71.39) (end 87.8573 72.8573) (width 0.5) (layer "B.Cu") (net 3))
 (segment (start 91.47 71.39) (end 91.1983 71.6617) (width 0.5) (layer "B.Cu") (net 28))
 (segment (start 94.01 71.39) (end 92.2553 73.1447) (width 0.5) (layer "B.Cu") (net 10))
 (segment (start 101.8205 134.6395) (end 101.8205 116.2005) (width 0.5) (layer "B.Cu") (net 2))
 (segment (start 120.8445 134.6155) (end 120.54 134.92) (width 0.5) (layer "B.Cu") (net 2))
 (segment (start 139.8514 154.2314) (end 139.8514 160.1381) (width 0.5) (layer "B.Cu") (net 2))
 (segment (start 139.54 115.92) (end 139.8205 116.2005) (width 0.5) (layer "B.Cu") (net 2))
 (segment (start 82.54 134.92) (end 82.8205 134.6395) (width 0.5) (layer "B.Cu") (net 2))
 (segment (start 63.8205 116.2005) (end 63.54 115.92) (width 0.5) (layer "B.Cu") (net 2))
 (segment (start 96.55 53.61) (end 98.3005 51.8595) (width 0.5) (layer "B.Cu") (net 2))
 (segment (start 63.887 153.92) (end 63.887 135.267) (width 0.5) (layer "B.Cu") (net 2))
 (segment (start 139.839 78.219) (end 139.839 96.621) (width 0.5) (layer "B.Cu") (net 2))
 (segment (start 63.839 78.219) (end 63.839 96.621) (width 0.5) (layer "B.Cu") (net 2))
 (segment (start 82.8321 154.2121) (end 82.54 153.92) (width 0.5) (layer "B.Cu") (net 2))
 (segment (start 101.839 78.219) (end 101.839 96.621) (width 0.5) (layer "B.Cu") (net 2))
 (segment (start 138.1537 161.8358) (end 120.8321 161.8358) (width 0.5) (layer "B.Cu") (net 2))
 (segment (start 113.4795 51.8595) (end 139.54 77.92) (width 0.5) (layer "B.Cu") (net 2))
 (segment (start 82.54 134.92) (end 82.8445 135.2245) (width 0.5) (layer "B.Cu") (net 2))
 (segment (start 98.3005 51.8595) (end 113.4795 51.8595) (width 0.5) (layer "B.Cu") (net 2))
 (segment (start 101.8205 97.2005) (end 101.54 96.92) (width 0.5) (layer "B.Cu") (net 2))
 (segment (start 63.839 96.621) (end 63.54 96.92) (width 0.5) (layer "B.Cu") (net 2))
 (segment (start 139.54 77.92) (end 139.839 78.219) (width 0.5) (layer "B.Cu") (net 2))
 (segment (start 139.839 96.621) (end 139.54 96.92) (width 0.5) (layer "B.Cu") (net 2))
 (segment (start 63.54 77.92) (end 63.839 78.219) (width 0.5) (layer "B.Cu") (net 2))
 (segment (start 120.8321 161.8358) (end 120.8321 154.2121) (width 0.5) (layer "B.Cu") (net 2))
 (segment (start 101.8321 153.6279) (end 101.54 153.92) (width 0.5) (layer "B.Cu") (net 2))
 (segment (start 101.8489 160.1994) (end 100.2236 161.8247) (width 0.5) (layer "B.Cu") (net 2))
 (segment (start 82.8514 115.6086) (end 82.54 115.92) (width 0.5) (layer "B.Cu") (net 2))
 (segment (start 82.839 78.219) (end 82.839 96.621) (width 0.5) (layer "B.Cu") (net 2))
 (segment (start 82.8445 135.2245) (end 82.8445 153.6155) (width 0.5) (layer "B.Cu") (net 2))
 (segment (start 82.8445 153.6155) (end 82.54 153.92) (width 0.5) (layer "B.Cu") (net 2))
 (segment (start 82.8205 116.2005) (end 82.54 115.92) (width 0.5) (layer "B.Cu") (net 2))
 (segment (start 63.8514 115.6086) (end 63.54 115.92) (width 0.5) (layer "B.Cu") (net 2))
 (segment (start 120.54 115.92) (end 120.8445 116.2245) (width 0.5) (layer "B.Cu") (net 2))
 (segment (start 139.54 96.92) (end 139.8514 97.2314) (width 0.5) (layer "B.Cu") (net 2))
 (segment (start 101.54 77.92) (end 101.839 78.219) (width 0.5) (layer "B.Cu") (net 2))
 (segment (start 101.54 115.92) (end 101.8205 115.6395) (width 0.5) (layer "B.Cu") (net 2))
 (segment (start 120.8535 135.2335) (end 120.8535 153.6065) (width 0.5) (layer "B.Cu") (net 2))
 (segment (start 101.839 96.621) (end 101.54 96.92) (width 0.5) (layer "B.Cu") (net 2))
 (segment (start 82.54 96.92) (end 82.8514 97.2314) (width 0.5) (layer "B.Cu") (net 2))
 (segment (start 120.8321 161.8358) (end 103.4853 161.8358) (width 0.5) (layer "B.Cu") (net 2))
 (segment (start 82.54 77.92) (end 82.839 78.219) (width 0.5) (layer "B.Cu") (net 2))
 (segment (start 139.8205 116.2005) (end 139.8205 134.6395) (width 0.5) (layer "B.Cu") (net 2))
 (segment (start 120.8321 154.2121) (end 120.54 153.92) (width 0.5) (layer "B.Cu") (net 2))
 (segment (start 120.54 77.92) (end 120.839 78.219) (width 0.5) (layer "B.Cu") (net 2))
 (segment (start 82.8514 97.2314) (end 82.8514 115.6086) (width 0.5) (layer "B.Cu") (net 2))
 (segment (start 101.8205 116.2005) (end 101.54 115.92) (width 0.5) (layer "B.Cu") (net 2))
 (segment (start 82.8321 161.8247) (end 82.8321 154.2121) (width 0.5) (layer "B.Cu") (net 2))
 (segment (start 82.839 96.621) (end 82.54 96.92) (width 0.5) (layer "B.Cu") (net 2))
 (segment (start 63.887 153.92) (end 63.54 153.92) (width 0.5) (layer "B.Cu") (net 2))
 (segment (start 63.887 135.267) (end 63.54 134.92) (width 0.5) (layer "B.Cu") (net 2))
 (segment (start 120.54 134.92) (end 120.8535 135.2335) (width 0.5) (layer "B.Cu") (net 2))
 (segment (start 120.8535 153.6065) (end 120.54 153.92) (width 0.5) (layer "B.Cu") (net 2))
 (segment (start 139.839 153.621) (end 139.839 135.219) (width 0.5) (layer "B.Cu") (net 2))
 (segment (start 139.54 153.92) (end 139.8514 154.2314) (width 0.5) (layer "B.Cu") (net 2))
 (segment (start 63.54 96.92) (end 63.8514 97.2314) (width 0.5) (layer "B.Cu") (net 2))
 (segment (start 103.4853 161.8358) (end 101.8489 160.1994) (width 0.5) (layer "B.Cu") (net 2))
 (segment (start 71.7917 161.8247) (end 82.8321 161.8247) (width 0.5) (layer "B.Cu") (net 2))
 (segment (start 139.8205 134.6395) (end 139.54 134.92) (width 0.5) (layer "B.Cu") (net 2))
 (segment (start 101.54 134.92) (end 101.8205 134.6395) (width 0.5) (layer "B.Cu") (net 2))
 (segment (start 63.54 134.92) (end 63.8205 134.6395) (width 0.5) (layer "B.Cu") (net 2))
 (segment (start 82.8205 134.6395) (end 82.8205 116.2005) (width 0.5) (layer "B.Cu") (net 2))
 (segment (start 63.887 153.92) (end 71.7917 161.8247) (width 0.5) (layer "B.Cu") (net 2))
 (segment (start 120.839 78.219) (end 120.839 96.621) (width 0.5) (layer "B.Cu") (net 2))
 (segment (start 139.8514 97.2314) (end 139.8514 115.6086) (width 0.5) (layer "B.Cu") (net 2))
 (segment (start 139.54 153.92) (end 139.839 153.621) (width 0.5) (layer "B.Cu") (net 2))
 (segment (start 101.54 134.92) (end 101.8321 135.2121) (width 0.5) (layer "B.Cu") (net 2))
 (segment (start 120.839 96.621) (end 120.54 96.92) (width 0.5) (layer "B.Cu") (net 2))
 (segment (start 101.54 153.92) (end 101.8489 154.2289) (width 0.5) (layer "B.Cu") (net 2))
 (segment (start 101.8489 154.2289) (end 101.8489 160.1994) (width 0.5) (layer "B.Cu") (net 2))
 (segment (start 63.8205 134.6395) (end 63.8205 116.2005) (width 0.5) (layer "B.Cu") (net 2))
 (segment (start 120.8205 115.6395) (end 120.8205 97.2005) (width 0.5) (layer "B.Cu") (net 2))
 (segment (start 139.8514 115.6086) (end 139.54 115.92) (width 0.5) (layer "B.Cu") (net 2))
 (segment (start 139.8514 160.1381) (end 138.1537 161.8358) (width 0.5) (layer "B.Cu") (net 2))
 (segment (start 139.839 135.219) (end 139.54 134.92) (width 0.5) (layer "B.Cu") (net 2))
 (segment (start 101.8321 135.2121) (end 101.8321 153.6279) (width 0.5) (layer "B.Cu") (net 2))
 (segment (start 120.54 115.92) (end 120.8205 115.6395) (width 0.5) (layer "B.Cu") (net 2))
 (segment (start 101.8205 115.6395) (end 101.8205 97.2005) (width 0.5) (layer "B.Cu") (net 2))
 (segment (start 120.8445 116.2245) (end 120.8445 134.6155) (width 0.5) (layer "B.Cu") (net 2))
 (segment (start 120.8205 97.2005) (end 120.54 96.92) (width 0.5) (layer "B.Cu") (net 2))
 (segment (start 63.8514 97.2314) (end 63.8514 115.6086) (width 0.5) (layer "B.Cu") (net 2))
 (segment (start 100.2236 161.8247) (end 82.8321 161.8247) (width 0.5) (layer "B.Cu") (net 2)))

